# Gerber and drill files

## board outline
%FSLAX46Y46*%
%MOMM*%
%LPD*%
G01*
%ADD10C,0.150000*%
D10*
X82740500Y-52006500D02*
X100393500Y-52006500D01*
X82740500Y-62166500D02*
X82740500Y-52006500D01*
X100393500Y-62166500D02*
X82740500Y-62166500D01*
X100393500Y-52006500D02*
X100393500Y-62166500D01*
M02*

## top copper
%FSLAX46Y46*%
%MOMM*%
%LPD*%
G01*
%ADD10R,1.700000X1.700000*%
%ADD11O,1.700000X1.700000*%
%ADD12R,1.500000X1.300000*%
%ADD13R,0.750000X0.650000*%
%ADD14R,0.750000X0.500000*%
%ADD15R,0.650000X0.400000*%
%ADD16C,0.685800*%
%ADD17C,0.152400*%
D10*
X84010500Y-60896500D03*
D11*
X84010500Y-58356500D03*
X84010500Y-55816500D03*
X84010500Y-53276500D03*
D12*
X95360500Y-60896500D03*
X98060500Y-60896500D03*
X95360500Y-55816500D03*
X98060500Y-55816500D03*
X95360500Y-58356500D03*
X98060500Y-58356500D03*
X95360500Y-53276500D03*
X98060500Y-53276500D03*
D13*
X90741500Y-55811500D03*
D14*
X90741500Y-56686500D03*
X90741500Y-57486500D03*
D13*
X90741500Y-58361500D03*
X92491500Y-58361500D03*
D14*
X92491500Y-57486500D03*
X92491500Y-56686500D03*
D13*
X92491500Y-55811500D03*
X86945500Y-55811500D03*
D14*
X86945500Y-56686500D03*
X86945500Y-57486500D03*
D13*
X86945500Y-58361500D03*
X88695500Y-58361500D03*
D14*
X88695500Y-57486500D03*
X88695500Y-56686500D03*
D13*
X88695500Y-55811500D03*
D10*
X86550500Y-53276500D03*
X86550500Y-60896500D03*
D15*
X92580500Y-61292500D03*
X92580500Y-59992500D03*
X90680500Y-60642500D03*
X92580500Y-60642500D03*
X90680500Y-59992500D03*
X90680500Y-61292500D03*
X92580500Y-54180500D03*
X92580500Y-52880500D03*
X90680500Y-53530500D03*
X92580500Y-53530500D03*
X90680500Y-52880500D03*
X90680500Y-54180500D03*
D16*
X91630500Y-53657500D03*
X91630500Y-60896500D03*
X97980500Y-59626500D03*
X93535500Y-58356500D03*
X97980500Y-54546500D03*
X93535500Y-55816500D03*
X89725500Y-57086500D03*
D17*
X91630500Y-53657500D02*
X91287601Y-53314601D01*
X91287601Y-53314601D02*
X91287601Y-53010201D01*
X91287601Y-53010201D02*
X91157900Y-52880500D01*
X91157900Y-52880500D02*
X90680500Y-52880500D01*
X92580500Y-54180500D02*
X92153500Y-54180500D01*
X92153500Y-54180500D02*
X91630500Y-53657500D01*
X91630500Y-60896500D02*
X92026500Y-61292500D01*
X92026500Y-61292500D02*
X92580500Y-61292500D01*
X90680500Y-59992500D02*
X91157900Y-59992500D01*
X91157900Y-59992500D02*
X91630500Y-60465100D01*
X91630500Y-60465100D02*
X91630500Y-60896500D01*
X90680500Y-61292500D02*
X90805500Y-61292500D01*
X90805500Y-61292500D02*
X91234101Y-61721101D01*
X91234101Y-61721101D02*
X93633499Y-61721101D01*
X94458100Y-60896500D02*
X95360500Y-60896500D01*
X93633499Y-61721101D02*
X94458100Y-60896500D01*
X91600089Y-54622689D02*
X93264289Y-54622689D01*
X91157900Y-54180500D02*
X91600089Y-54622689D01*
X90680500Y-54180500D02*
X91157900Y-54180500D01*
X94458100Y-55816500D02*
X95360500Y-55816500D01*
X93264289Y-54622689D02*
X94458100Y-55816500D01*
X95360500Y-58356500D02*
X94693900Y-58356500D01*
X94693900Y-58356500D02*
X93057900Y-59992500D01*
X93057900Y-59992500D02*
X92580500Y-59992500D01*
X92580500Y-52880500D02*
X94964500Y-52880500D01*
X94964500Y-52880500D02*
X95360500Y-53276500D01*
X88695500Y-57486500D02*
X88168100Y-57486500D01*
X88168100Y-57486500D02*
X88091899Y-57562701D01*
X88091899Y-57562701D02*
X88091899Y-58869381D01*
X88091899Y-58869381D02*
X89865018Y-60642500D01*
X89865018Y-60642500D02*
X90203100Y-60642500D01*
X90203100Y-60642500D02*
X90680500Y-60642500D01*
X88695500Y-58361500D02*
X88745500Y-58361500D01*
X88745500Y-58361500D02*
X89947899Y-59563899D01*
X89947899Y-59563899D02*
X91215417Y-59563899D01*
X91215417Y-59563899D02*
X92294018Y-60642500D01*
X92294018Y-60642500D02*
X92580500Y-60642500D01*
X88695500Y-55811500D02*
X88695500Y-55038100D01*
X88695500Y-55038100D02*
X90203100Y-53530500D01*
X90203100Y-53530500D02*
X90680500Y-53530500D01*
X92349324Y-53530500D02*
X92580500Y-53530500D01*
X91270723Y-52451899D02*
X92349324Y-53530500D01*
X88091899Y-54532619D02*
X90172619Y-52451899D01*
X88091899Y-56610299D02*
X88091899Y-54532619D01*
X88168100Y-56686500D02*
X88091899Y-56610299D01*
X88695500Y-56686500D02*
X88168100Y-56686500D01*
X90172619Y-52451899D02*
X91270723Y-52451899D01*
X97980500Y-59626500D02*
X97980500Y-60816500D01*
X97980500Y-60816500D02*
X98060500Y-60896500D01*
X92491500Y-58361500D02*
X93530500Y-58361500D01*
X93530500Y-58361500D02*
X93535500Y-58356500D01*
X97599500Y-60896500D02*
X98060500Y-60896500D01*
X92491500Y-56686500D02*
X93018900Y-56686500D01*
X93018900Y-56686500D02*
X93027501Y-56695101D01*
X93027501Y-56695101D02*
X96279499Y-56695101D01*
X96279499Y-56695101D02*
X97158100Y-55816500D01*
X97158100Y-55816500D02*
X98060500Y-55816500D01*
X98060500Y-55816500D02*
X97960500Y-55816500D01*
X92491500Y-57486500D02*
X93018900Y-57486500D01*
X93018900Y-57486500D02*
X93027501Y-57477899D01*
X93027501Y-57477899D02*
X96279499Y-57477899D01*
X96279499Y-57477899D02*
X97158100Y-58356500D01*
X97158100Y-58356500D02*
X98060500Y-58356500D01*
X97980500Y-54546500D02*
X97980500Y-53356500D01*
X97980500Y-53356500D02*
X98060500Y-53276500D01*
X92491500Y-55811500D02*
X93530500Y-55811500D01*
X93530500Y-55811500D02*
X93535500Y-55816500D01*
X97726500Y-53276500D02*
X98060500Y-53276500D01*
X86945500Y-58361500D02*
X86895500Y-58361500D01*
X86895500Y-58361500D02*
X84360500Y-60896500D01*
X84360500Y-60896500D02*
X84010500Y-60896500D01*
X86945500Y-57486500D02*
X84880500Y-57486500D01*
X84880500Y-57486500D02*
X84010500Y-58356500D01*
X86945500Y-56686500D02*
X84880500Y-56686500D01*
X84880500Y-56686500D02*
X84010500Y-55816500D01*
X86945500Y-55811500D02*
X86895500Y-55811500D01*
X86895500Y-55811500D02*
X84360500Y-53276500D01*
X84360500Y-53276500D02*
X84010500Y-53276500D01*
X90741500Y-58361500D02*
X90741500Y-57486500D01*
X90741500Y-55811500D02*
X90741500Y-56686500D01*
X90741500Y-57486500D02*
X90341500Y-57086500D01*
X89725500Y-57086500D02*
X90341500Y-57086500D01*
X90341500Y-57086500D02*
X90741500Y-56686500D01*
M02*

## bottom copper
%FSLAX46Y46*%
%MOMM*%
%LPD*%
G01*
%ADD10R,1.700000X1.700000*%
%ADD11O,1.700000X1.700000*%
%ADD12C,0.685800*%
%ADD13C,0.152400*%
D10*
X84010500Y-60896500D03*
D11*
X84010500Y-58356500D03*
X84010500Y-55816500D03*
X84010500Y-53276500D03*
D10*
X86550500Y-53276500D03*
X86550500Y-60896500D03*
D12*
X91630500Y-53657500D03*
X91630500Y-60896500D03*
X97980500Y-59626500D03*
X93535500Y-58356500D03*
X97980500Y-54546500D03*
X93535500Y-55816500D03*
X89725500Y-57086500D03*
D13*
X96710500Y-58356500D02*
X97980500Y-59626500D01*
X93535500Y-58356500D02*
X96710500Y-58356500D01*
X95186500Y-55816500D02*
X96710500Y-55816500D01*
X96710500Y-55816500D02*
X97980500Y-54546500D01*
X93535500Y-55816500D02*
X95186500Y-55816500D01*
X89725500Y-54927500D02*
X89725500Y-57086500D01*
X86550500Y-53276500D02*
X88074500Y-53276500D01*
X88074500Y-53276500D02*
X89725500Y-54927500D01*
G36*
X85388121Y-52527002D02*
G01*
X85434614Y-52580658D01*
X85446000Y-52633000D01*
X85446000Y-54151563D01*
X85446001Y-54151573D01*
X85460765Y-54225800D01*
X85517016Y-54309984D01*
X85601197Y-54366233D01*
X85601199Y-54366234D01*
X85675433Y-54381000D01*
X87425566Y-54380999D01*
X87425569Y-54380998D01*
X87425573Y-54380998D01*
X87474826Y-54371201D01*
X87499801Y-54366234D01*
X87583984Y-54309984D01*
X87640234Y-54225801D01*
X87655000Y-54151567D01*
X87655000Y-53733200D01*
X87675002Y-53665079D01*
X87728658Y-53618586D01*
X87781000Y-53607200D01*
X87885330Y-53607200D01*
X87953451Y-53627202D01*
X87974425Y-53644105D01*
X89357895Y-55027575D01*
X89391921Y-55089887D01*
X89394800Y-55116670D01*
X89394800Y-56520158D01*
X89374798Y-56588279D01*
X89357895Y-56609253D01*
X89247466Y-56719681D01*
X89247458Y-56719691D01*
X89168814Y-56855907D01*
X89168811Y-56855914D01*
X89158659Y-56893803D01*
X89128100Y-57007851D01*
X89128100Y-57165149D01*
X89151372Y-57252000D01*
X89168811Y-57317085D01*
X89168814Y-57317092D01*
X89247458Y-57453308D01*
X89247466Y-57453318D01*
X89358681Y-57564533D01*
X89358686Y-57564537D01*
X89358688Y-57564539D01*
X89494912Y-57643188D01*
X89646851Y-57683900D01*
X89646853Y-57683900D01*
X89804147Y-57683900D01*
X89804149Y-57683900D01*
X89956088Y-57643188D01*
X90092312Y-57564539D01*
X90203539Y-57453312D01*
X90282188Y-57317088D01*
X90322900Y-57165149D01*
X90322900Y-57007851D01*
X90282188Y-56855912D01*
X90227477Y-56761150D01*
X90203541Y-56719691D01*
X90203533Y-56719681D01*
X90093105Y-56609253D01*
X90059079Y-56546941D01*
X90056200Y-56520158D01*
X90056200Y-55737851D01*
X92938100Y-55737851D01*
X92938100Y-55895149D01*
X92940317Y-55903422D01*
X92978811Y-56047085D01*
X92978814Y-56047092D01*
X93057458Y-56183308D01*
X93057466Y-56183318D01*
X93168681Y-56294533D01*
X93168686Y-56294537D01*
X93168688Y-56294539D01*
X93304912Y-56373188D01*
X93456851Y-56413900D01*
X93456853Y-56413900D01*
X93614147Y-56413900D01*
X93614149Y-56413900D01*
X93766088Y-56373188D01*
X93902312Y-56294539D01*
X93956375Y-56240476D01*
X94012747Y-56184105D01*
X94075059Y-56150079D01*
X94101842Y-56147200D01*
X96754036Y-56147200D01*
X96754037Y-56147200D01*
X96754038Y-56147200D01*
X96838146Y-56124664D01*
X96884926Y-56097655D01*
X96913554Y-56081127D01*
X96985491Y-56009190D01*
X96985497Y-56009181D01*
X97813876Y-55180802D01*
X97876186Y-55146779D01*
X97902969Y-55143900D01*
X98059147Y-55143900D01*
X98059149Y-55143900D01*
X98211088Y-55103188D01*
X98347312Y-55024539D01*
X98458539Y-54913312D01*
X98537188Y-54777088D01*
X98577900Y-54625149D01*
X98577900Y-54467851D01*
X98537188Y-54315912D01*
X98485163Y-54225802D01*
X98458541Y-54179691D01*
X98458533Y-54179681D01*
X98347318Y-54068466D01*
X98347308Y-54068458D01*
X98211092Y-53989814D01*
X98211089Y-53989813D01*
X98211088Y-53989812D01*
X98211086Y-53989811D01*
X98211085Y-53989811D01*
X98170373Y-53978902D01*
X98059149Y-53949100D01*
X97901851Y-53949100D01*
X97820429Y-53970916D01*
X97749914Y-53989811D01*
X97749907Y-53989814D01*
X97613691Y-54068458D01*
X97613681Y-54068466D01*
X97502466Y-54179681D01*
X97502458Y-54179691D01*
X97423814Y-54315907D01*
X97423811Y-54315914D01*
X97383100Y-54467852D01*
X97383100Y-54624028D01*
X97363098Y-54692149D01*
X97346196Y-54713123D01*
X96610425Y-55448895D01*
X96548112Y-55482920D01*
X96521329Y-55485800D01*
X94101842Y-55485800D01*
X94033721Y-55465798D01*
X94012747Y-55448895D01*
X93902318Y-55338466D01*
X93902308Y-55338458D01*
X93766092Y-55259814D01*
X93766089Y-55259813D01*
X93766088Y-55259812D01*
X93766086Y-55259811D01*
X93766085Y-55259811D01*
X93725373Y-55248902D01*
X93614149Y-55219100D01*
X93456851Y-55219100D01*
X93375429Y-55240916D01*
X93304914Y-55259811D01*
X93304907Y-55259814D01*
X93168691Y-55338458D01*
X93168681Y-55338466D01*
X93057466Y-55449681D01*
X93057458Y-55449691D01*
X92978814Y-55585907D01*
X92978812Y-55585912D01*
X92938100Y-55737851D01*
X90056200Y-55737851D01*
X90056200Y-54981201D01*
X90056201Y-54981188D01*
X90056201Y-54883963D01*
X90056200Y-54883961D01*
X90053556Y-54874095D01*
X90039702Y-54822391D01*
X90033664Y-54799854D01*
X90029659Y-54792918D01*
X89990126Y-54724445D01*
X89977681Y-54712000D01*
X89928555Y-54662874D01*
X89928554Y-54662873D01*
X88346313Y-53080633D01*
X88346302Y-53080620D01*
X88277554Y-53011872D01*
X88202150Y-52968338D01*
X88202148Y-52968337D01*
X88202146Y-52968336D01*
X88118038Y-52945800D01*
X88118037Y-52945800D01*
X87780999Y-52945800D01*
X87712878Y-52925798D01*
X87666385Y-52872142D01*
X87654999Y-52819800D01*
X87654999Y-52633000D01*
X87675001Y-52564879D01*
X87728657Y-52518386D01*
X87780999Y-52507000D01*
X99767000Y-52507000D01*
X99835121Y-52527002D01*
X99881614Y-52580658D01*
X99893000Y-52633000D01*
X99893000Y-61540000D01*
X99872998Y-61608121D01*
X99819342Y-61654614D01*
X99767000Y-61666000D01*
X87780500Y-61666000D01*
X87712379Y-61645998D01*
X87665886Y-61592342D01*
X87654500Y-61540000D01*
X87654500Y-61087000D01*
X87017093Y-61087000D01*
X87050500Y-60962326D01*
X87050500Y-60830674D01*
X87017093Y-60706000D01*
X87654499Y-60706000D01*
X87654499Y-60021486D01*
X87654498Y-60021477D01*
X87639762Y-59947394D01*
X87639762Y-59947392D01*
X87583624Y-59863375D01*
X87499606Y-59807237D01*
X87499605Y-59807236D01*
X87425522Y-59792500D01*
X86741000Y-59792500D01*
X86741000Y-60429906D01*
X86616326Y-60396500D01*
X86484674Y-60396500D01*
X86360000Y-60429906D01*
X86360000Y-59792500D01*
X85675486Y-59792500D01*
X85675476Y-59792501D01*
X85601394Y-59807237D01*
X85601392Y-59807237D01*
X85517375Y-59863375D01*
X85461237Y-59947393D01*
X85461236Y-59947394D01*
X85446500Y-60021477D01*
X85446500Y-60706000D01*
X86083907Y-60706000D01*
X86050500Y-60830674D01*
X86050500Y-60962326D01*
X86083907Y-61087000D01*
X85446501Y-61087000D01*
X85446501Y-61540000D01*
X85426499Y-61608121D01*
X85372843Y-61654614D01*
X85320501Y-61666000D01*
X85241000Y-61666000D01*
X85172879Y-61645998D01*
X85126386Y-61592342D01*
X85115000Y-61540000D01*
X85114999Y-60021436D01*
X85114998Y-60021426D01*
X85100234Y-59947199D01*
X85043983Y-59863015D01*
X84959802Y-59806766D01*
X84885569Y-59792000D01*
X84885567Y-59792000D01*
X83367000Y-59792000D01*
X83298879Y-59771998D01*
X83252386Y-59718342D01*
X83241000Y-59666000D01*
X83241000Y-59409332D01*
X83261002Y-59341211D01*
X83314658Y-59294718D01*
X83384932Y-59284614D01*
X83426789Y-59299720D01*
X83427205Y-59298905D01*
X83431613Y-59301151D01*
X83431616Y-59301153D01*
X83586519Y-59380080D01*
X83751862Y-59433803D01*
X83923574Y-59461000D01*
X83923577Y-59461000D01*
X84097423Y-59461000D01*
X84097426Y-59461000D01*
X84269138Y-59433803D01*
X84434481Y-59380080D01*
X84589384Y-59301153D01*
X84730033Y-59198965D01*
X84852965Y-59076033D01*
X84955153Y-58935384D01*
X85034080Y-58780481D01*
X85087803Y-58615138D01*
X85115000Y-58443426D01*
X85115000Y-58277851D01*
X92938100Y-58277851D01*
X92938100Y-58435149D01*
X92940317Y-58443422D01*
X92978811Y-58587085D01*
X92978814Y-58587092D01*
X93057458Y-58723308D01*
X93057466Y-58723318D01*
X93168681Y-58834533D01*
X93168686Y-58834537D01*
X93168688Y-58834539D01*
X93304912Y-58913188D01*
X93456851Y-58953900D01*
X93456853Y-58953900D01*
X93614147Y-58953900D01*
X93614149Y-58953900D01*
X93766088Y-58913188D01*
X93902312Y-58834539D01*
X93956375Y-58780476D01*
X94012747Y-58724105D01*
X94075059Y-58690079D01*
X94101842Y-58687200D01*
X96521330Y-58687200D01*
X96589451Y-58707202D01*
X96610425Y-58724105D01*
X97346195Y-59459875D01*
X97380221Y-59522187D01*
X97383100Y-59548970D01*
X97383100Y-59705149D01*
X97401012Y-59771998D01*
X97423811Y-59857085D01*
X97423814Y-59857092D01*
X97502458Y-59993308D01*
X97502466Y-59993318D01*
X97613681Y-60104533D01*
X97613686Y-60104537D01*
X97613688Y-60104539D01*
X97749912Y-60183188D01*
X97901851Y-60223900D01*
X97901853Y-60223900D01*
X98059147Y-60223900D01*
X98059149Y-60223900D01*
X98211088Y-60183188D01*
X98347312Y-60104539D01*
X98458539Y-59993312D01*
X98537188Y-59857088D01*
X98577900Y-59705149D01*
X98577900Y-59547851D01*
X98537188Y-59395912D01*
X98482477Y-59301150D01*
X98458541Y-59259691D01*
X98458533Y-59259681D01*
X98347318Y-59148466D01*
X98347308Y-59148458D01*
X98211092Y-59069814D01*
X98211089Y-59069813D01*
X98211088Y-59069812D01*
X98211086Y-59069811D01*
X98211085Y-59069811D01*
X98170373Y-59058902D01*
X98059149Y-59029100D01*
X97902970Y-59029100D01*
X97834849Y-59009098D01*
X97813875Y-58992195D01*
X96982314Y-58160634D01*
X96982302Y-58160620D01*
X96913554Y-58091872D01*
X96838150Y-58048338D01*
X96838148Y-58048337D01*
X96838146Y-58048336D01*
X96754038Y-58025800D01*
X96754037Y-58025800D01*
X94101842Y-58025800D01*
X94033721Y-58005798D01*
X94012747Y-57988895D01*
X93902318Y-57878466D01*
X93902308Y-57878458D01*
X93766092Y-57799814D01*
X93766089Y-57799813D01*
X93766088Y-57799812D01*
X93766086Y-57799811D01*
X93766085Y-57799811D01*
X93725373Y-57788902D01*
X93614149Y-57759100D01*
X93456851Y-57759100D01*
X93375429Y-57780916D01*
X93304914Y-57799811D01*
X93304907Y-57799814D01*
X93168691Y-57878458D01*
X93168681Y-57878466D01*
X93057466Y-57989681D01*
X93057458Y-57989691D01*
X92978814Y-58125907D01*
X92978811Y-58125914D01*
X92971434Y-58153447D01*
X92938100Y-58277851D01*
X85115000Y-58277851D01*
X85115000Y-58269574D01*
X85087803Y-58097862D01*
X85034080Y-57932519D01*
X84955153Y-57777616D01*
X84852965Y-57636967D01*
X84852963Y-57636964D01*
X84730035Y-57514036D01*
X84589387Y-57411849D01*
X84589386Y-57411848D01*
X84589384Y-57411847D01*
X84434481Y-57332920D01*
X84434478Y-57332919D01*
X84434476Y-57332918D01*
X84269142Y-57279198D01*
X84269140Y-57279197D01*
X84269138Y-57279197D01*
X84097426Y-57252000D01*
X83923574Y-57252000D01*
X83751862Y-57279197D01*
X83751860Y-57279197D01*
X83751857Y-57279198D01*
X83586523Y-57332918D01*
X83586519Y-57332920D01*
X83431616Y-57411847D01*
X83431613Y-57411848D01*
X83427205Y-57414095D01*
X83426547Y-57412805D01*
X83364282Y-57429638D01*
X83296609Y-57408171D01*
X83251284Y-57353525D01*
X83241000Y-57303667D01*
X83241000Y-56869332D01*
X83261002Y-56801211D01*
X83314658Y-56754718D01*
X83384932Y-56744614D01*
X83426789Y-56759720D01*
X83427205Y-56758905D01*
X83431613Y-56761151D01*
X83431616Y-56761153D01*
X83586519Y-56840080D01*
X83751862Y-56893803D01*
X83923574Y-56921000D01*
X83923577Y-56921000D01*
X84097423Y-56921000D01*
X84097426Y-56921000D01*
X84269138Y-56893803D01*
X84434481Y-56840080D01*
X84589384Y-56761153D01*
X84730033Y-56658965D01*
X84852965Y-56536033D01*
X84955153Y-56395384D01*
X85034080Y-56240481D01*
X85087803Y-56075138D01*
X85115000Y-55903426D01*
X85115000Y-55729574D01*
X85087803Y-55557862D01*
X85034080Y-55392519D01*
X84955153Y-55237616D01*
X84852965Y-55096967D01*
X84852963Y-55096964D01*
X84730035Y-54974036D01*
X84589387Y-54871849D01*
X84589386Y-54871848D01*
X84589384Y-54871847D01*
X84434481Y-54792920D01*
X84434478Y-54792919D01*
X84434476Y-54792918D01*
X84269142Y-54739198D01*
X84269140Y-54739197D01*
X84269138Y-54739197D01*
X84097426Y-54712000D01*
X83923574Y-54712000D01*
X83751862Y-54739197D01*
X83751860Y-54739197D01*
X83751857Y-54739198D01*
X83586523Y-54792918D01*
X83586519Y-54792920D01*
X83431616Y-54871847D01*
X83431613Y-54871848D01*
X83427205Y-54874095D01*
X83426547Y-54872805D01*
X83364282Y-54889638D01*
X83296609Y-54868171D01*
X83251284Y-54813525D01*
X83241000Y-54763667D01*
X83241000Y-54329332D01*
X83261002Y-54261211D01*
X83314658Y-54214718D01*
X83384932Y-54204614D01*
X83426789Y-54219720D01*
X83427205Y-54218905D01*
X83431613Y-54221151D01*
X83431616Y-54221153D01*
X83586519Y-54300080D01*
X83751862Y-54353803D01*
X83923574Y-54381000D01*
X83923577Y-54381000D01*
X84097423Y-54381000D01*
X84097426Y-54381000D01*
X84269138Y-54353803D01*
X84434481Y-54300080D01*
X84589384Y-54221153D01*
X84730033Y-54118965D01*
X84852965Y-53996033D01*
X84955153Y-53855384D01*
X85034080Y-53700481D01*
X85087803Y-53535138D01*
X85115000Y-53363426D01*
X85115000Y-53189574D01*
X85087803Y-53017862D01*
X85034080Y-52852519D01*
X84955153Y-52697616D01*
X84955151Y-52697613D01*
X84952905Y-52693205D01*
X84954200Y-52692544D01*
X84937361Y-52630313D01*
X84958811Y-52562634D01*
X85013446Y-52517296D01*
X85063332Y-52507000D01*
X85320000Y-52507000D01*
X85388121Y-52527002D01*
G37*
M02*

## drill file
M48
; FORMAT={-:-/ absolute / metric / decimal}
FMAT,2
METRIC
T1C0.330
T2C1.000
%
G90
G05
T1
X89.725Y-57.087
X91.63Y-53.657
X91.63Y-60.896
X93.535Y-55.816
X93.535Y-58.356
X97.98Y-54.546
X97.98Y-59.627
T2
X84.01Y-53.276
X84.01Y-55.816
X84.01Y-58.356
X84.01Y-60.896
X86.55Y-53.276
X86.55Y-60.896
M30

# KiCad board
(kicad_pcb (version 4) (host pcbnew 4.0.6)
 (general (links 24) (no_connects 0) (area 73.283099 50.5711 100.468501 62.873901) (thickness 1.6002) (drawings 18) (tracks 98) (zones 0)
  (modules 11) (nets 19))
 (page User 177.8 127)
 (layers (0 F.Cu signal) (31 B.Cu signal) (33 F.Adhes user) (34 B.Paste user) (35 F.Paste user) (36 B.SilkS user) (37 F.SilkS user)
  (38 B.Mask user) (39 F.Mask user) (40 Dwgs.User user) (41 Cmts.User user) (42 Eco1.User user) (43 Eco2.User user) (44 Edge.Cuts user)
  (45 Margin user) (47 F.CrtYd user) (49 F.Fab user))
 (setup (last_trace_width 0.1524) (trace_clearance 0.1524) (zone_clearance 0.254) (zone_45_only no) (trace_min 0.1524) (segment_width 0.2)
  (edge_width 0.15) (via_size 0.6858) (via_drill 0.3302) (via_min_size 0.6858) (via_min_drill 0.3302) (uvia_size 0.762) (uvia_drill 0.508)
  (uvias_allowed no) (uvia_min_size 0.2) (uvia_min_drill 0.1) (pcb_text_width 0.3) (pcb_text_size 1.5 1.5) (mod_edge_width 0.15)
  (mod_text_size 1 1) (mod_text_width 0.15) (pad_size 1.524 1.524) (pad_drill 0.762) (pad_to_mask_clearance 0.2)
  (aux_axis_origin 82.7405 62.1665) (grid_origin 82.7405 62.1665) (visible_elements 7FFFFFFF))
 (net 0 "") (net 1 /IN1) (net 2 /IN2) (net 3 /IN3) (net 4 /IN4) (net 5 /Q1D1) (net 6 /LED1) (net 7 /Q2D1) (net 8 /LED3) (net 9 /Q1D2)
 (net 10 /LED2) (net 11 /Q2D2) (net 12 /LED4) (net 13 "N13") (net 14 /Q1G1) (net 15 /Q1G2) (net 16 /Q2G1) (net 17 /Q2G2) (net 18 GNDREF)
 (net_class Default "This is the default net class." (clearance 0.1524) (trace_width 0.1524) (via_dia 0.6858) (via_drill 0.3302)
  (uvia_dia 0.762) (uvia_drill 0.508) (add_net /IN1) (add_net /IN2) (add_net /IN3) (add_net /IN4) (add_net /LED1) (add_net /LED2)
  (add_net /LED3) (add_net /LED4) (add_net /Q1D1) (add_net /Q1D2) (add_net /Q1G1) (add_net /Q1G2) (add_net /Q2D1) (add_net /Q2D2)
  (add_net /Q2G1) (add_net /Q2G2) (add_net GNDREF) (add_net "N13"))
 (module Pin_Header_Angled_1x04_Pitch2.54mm (layer F.Cu) (at 84.0105 60.8965 180)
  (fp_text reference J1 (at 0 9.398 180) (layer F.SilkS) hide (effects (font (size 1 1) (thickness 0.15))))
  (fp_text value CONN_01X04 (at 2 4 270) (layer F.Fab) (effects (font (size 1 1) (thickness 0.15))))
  (pad 1 thru_hole rect (at 0 0 180) (size 1.7 1.7) (drill 1) (layers *.Cu *.Mask) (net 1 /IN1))
  (pad 2 thru_hole oval (at 0 2.54 180) (size 1.7 1.7) (drill 1) (layers *.Cu *.Mask) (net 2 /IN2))
  (pad 3 thru_hole oval (at 0 5.08 180) (size 1.7 1.7) (drill 1) (layers *.Cu *.Mask) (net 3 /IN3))
  (pad 4 thru_hole oval (at 0 7.62 180) (size 1.7 1.7) (drill 1) (layers *.Cu *.Mask) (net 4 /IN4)))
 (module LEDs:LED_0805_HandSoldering (layer F.Cu) (at 96.7105 60.8965)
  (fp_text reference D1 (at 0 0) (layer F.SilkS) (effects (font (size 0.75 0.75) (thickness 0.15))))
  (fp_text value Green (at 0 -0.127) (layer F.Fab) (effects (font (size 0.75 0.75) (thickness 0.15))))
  (pad 1 smd rect (at -1.35 0) (size 1.5 1.3) (layers F.Cu F.Paste F.Mask) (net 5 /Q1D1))
  (pad 2 smd rect (at 1.35 0) (size 1.5 1.3) (layers F.Cu F.Paste F.Mask) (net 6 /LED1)))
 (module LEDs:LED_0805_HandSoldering (layer F.Cu) (at 96.7105 55.8165)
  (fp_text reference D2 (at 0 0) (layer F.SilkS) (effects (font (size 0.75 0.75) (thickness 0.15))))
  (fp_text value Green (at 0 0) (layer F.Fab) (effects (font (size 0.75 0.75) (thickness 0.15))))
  (pad 1 smd rect (at -1.35 0) (size 1.5 1.3) (layers F.Cu F.Paste F.Mask) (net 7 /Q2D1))
  (pad 2 smd rect (at 1.35 0) (size 1.5 1.3) (layers F.Cu F.Paste F.Mask) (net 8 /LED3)))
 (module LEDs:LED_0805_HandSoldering (layer F.Cu) (at 96.7105 58.3565)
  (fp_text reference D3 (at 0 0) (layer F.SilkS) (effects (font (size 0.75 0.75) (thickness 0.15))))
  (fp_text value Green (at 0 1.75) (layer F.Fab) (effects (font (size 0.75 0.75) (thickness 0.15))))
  (pad 1 smd rect (at -1.35 0) (size 1.5 1.3) (layers F.Cu F.Paste F.Mask) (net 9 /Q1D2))
  (pad 2 smd rect (at 1.35 0) (size 1.5 1.3) (layers F.Cu F.Paste F.Mask) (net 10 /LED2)))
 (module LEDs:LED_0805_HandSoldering (layer F.Cu) (at 96.7105 53.2765)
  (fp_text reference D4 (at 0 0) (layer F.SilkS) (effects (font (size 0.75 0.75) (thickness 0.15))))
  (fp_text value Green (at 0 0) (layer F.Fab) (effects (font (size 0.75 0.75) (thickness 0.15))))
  (pad 1 smd rect (at -1.35 0) (size 1.5 1.3) (layers F.Cu F.Paste F.Mask) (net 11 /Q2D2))
  (pad 2 smd rect (at 1.35 0) (size 1.5 1.3) (layers F.Cu F.Paste F.Mask) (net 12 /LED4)))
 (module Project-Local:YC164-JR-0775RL (layer F.Cu) (at 91.6165 57.0865)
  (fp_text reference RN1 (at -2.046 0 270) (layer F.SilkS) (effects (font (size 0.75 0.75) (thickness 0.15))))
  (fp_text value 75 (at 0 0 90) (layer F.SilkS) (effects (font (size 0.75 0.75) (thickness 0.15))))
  (pad 1 smd rect (at -0.875 -1.275) (size 0.75 0.65) (layers F.Cu F.Paste F.Mask) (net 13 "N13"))
  (pad 2 smd rect (at -0.875 -0.4) (size 0.75 0.5) (layers F.Cu F.Paste F.Mask) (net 13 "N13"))
  (pad 3 smd rect (at -0.875 0.4) (size 0.75 0.5) (layers F.Cu F.Paste F.Mask) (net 13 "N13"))
  (pad 4 smd rect (at -0.875 1.275) (size 0.75 0.65) (layers F.Cu F.Paste F.Mask) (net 13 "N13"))
  (pad 5 smd rect (at 0.875 1.275) (size 0.75 0.65) (layers F.Cu F.Paste F.Mask) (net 6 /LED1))
  (pad 6 smd rect (at 0.875 0.4) (size 0.75 0.5) (layers F.Cu F.Paste F.Mask) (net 10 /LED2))
  (pad 7 smd rect (at 0.875 -0.4) (size 0.75 0.5) (layers F.Cu F.Paste F.Mask) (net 8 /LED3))
  (pad 8 smd rect (at 0.875 -1.275) (size 0.75 0.65) (layers F.Cu F.Paste F.Mask) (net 12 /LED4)))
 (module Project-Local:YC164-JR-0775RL (layer F.Cu) (at 87.8205 57.0865)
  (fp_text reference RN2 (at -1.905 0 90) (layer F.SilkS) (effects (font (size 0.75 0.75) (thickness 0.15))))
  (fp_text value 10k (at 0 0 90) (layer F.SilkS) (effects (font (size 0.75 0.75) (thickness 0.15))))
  (pad 1 smd rect (at -0.875 -1.275) (size 0.75 0.65) (layers F.Cu F.Paste F.Mask) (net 4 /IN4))
  (pad 2 smd rect (at -0.875 -0.4) (size 0.75 0.5) (layers F.Cu F.Paste F.Mask) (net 3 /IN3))
  (pad 3 smd rect (at -0.875 0.4) (size 0.75 0.5) (layers F.Cu F.Paste F.Mask) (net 2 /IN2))
  (pad 4 smd rect (at -0.875 1.275) (size 0.75 0.65) (layers F.Cu F.Paste F.Mask) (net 1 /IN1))
  (pad 5 smd rect (at 0.875 1.275) (size 0.75 0.65) (layers F.Cu F.Paste F.Mask) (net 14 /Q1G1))
  (pad 6 smd rect (at 0.875 0.4) (size 0.75 0.5) (layers F.Cu F.Paste F.Mask) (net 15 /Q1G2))
  (pad 7 smd rect (at 0.875 -0.4) (size 0.75 0.5) (layers F.Cu F.Paste F.Mask) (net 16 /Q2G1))
  (pad 8 smd rect (at 0.875 -1.275) (size 0.75 0.65) (layers F.Cu F.Paste F.Mask) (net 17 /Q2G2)))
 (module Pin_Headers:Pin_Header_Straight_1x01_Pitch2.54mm (layer F.Cu) (at 86.5505 53.2765)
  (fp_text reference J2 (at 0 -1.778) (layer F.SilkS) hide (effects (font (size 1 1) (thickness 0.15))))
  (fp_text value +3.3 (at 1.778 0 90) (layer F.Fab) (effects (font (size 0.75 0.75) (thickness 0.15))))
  (pad 1 thru_hole rect (at 0 0) (size 1.7 1.7) (drill 1) (layers *.Cu *.Mask) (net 13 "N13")))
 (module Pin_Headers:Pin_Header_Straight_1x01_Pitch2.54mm (layer F.Cu) (at 86.5505 60.8965)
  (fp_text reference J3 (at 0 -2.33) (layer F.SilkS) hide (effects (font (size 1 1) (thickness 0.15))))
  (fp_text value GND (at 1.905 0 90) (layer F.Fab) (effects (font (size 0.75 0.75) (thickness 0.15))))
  (pad 1 thru_hole rect (at 0 0) (size 1.7 1.7) (drill 1) (layers *.Cu *.Mask) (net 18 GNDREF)))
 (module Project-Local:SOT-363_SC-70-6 (layer F.Cu) (at 91.6305 60.6425 180)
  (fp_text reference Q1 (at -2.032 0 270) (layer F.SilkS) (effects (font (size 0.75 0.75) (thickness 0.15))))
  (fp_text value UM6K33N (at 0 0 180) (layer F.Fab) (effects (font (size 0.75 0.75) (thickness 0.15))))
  (pad 1 smd rect (at -0.95 -0.65 180) (size 0.65 0.4) (layers F.Cu F.Paste F.Mask) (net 18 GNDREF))
  (pad 3 smd rect (at -0.95 0.65 180) (size 0.65 0.4) (layers F.Cu F.Paste F.Mask) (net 9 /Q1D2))
  (pad 5 smd rect (at 0.95 0 180) (size 0.65 0.4) (layers F.Cu F.Paste F.Mask) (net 15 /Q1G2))
  (pad 2 smd rect (at -0.95 0 180) (size 0.65 0.4) (layers F.Cu F.Paste F.Mask) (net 14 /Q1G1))
  (pad 4 smd rect (at 0.95 0.65 180) (size 0.65 0.4) (layers F.Cu F.Paste F.Mask) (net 18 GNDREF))
  (pad 6 smd rect (at 0.95 -0.65 180) (size 0.65 0.4) (layers F.Cu F.Paste F.Mask) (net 5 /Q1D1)))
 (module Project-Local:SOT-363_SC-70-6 (layer F.Cu) (at 91.6305 53.5305 180)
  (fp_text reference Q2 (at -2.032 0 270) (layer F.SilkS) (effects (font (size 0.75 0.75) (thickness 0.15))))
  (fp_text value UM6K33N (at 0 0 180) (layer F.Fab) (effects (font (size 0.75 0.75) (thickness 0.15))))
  (pad 1 smd rect (at -0.95 -0.65 180) (size 0.65 0.4) (layers F.Cu F.Paste F.Mask) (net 18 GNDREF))
  (pad 3 smd rect (at -0.95 0.65 180) (size 0.65 0.4) (layers F.Cu F.Paste F.Mask) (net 11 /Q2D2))
  (pad 5 smd rect (at 0.95 0 180) (size 0.65 0.4) (layers F.Cu F.Paste F.Mask) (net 17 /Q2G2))
  (pad 2 smd rect (at -0.95 0 180) (size 0.65 0.4) (layers F.Cu F.Paste F.Mask) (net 16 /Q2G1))
  (pad 4 smd rect (at 0.95 0.65 180) (size 0.65 0.4) (layers F.Cu F.Paste F.Mask) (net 18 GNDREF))
  (pad 6 smd rect (at 0.95 -0.65 180) (size 0.65 0.4) (layers F.Cu F.Paste F.Mask) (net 7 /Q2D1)))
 (gr_line (start 82.7405 52.0065) (end 100.3935 52.0065) (layer Edge.Cuts) (width 0.15))
 (gr_line (start 82.7405 62.1665) (end 82.7405 52.0065) (layer Edge.Cuts) (width 0.15))
 (gr_line (start 100.3935 62.1665) (end 82.7405 62.1665) (layer Edge.Cuts) (width 0.15))
 (gr_line (start 100.3935 52.0065) (end 100.3935 62.1665) (layer Edge.Cuts) (width 0.15))
 (segment (start 91.6305 53.6575) (end 91.287601 53.314601) (width 0.1524) (layer F.Cu) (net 18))
 (segment (start 91.287601 53.314601) (end 91.287601 53.010201) (width 0.1524) (layer F.Cu) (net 18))
 (segment (start 91.287601 53.010201) (end 91.1579 52.8805) (width 0.1524) (layer F.Cu) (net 18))
 (segment (start 91.1579 52.8805) (end 90.6805 52.8805) (width 0.1524) (layer F.Cu) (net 18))
 (segment (start 92.5805 54.1805) (end 92.1535 54.1805) (width 0.1524) (layer F.Cu) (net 18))
 (segment (start 92.1535 54.1805) (end 91.6305 53.6575) (width 0.1524) (layer F.Cu) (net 18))
 (via (at 91.6305 53.6575) (size 0.6858) (drill 0.3302) (layers F.Cu B.Cu) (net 18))
 (segment (start 91.6305 60.8965) (end 92.0265 61.2925) (width 0.1524) (layer F.Cu) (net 18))
 (segment (start 92.0265 61.2925) (end 92.5805 61.2925) (width 0.1524) (layer F.Cu) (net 18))
 (via (at 91.6305 60.8965) (size 0.6858) (drill 0.3302) (layers F.Cu B.Cu) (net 18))
 (segment (start 90.6805 59.9925) (end 91.1579 59.9925) (width 0.1524) (layer F.Cu) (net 18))
 (segment (start 91.1579 59.9925) (end 91.6305 60.4651) (width 0.1524) (layer F.Cu) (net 18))
 (segment (start 91.6305 60.4651) (end 91.6305 60.8965) (width 0.1524) (layer F.Cu) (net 18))
 (segment (start 90.6805 61.2925) (end 90.8055 61.2925) (width 0.1524) (layer F.Cu) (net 5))
 (segment (start 90.8055 61.2925) (end 91.234101 61.721101) (width 0.1524) (layer F.Cu) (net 5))
 (segment (start 91.234101 61.721101) (end 93.633499 61.721101) (width 0.1524) (layer F.Cu) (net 5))
 (segment (start 94.4581 60.8965) (end 95.3605 60.8965) (width 0.1524) (layer F.Cu) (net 5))
 (segment (start 93.633499 61.721101) (end 94.4581 60.8965) (width 0.1524) (layer F.Cu) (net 5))
 (segment (start 91.600089 54.622689) (end 93.264289 54.622689) (width 0.1524) (layer F.Cu) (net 7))
 (segment (start 91.1579 54.1805) (end 91.600089 54.622689) (width 0.1524) (layer F.Cu) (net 7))
 (segment (start 90.6805 54.1805) (end 91.1579 54.1805) (width 0.1524) (layer F.Cu) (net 7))
 (segment (start 94.4581 55.8165) (end 95.3605 55.8165) (width 0.1524) (layer F.Cu) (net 7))
 (segment (start 93.264289 54.622689) (end 94.4581 55.8165) (width 0.1524) (layer F.Cu) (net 7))
 (segment (start 95.3605 58.3565) (end 94.6939 58.3565) (width 0.1524) (layer F.Cu) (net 9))
 (segment (start 94.6939 58.3565) (end 93.0579 59.9925) (width 0.1524) (layer F.Cu) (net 9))
 (segment (start 93.0579 59.9925) (end 92.5805 59.9925) (width 0.1524) (layer F.Cu) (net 9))
 (segment (start 92.5805 52.8805) (end 94.9645 52.8805) (width 0.1524) (layer F.Cu) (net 11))
 (segment (start 94.9645 52.8805) (end 95.3605 53.2765) (width 0.1524) (layer F.Cu) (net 11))
 (segment (start 88.6955 57.4865) (end 88.1681 57.4865) (width 0.1524) (layer F.Cu) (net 15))
 (segment (start 88.1681 57.4865) (end 88.091899 57.562701) (width 0.1524) (layer F.Cu) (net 15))
 (segment (start 88.091899 57.562701) (end 88.091899 58.869381) (width 0.1524) (layer F.Cu) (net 15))
 (segment (start 88.091899 58.869381) (end 89.865018 60.6425) (width 0.1524) (layer F.Cu) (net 15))
 (segment (start 89.865018 60.6425) (end 90.2031 60.6425) (width 0.1524) (layer F.Cu) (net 15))
 (segment (start 90.2031 60.6425) (end 90.6805 60.6425) (width 0.1524) (layer F.Cu) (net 15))
 (segment (start 88.6955 58.3615) (end 88.7455 58.3615) (width 0.1524) (layer F.Cu) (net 14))
 (segment (start 88.7455 58.3615) (end 89.947899 59.563899) (width 0.1524) (layer F.Cu) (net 14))
 (segment (start 89.947899 59.563899) (end 91.215417 59.563899) (width 0.1524) (layer F.Cu) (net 14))
 (segment (start 91.215417 59.563899) (end 92.294018 60.6425) (width 0.1524) (layer F.Cu) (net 14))
 (segment (start 92.294018 60.6425) (end 92.5805 60.6425) (width 0.1524) (layer F.Cu) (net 14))
 (segment (start 88.6955 55.8115) (end 88.6955 55.0381) (width 0.1524) (layer F.Cu) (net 17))
 (segment (start 88.6955 55.0381) (end 90.2031 53.5305) (width 0.1524) (layer F.Cu) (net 17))
 (segment (start 90.2031 53.5305) (end 90.6805 53.5305) (width 0.1524) (layer F.Cu) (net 17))
 (segment (start 92.349324 53.5305) (end 92.5805 53.5305) (width 0.1524) (layer F.Cu) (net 16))
 (segment (start 91.270723 52.451899) (end 92.349324 53.5305) (width 0.1524) (layer F.Cu) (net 16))
 (segment (start 88.091899 54.532619) (end 90.172619 52.451899) (width 0.1524) (layer F.Cu) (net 16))
 (segment (start 88.091899 56.610299) (end 88.091899 54.532619) (width 0.1524) (layer F.Cu) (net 16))
 (segment (start 88.1681 56.6865) (end 88.091899 56.610299) (width 0.1524) (layer F.Cu) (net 16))
 (segment (start 88.6955 56.6865) (end 88.1681 56.6865) (width 0.1524) (layer F.Cu) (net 16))
 (segment (start 90.172619 52.451899) (end 91.270723 52.451899) (width 0.1524) (layer F.Cu) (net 16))
 (segment (start 97.9805 59.6265) (end 97.9805 60.8165) (width 0.1524) (layer F.Cu) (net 6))
 (segment (start 97.9805 60.8165) (end 98.0605 60.8965) (width 0.1524) (layer F.Cu) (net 6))
 (via (at 97.9805 59.6265) (size 0.6858) (drill 0.3302) (layers F.Cu B.Cu) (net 6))
 (segment (start 96.7105 58.3565) (end 97.9805 59.6265) (width 0.1524) (layer B.Cu) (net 6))
 (segment (start 93.5355 58.3565) (end 96.7105 58.3565) (width 0.1524) (layer B.Cu) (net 6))
 (segment (start 92.4915 58.3615) (end 93.5305 58.3615) (width 0.1524) (layer F.Cu) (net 6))
 (segment (start 93.5305 58.3615) (end 93.5355 58.3565) (width 0.1524) (layer F.Cu) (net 6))
 (via (at 93.5355 58.3565) (size 0.6858) (drill 0.3302) (layers F.Cu B.Cu) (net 6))
 (segment (start 97.5995 60.8965) (end 98.0605 60.8965) (width 0.1524) (layer F.Cu) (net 6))
 (segment (start 92.4915 56.6865) (end 93.0189 56.6865) (width 0.1524) (layer F.Cu) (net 8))
 (segment (start 93.0189 56.6865) (end 93.027501 56.695101) (width 0.1524) (layer F.Cu) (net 8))
 (segment (start 93.027501 56.695101) (end 96.279499 56.695101) (width 0.1524) (layer F.Cu) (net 8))
 (segment (start 96.279499 56.695101) (end 97.1581 55.8165) (width 0.1524) (layer F.Cu) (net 8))
 (segment (start 97.1581 55.8165) (end 98.0605 55.8165) (width 0.1524) (layer F.Cu) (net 8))
 (segment (start 98.0605 55.8165) (end 97.9605 55.8165) (width 0.1524) (layer F.Cu) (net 8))
 (segment (start 92.4915 57.4865) (end 93.0189 57.4865) (width 0.1524) (layer F.Cu) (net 10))
 (segment (start 93.0189 57.4865) (end 93.027501 57.477899) (width 0.1524) (layer F.Cu) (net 10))
 (segment (start 93.027501 57.477899) (end 96.279499 57.477899) (width 0.1524) (layer F.Cu) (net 10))
 (segment (start 96.279499 57.477899) (end 97.1581 58.3565) (width 0.1524) (layer F.Cu) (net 10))
 (segment (start 97.1581 58.3565) (end 98.0605 58.3565) (width 0.1524) (layer F.Cu) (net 10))
 (segment (start 97.9805 54.5465) (end 97.9805 53.3565) (width 0.1524) (layer F.Cu) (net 12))
 (segment (start 97.9805 53.3565) (end 98.0605 53.2765) (width 0.1524) (layer F.Cu) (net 12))
 (segment (start 95.1865 55.8165) (end 96.7105 55.8165) (width 0.1524) (layer B.Cu) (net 12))
 (segment (start 96.7105 55.8165) (end 97.9805 54.5465) (width 0.1524) (layer B.Cu) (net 12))
 (via (at 97.9805 54.5465) (size 0.6858) (drill 0.3302) (layers F.Cu B.Cu) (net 12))
 (segment (start 93.5355 55.8165) (end 95.1865 55.8165) (width 0.1524) (layer B.Cu) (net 12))
 (segment (start 92.4915 55.8115) (end 93.5305 55.8115) (width 0.1524) (layer F.Cu) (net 12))
 (segment (start 93.5305 55.8115) (end 93.5355 55.8165) (width 0.1524) (layer F.Cu) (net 12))
 (via (at 93.5355 55.8165) (size 0.6858) (drill 0.3302) (layers F.Cu B.Cu) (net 12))
 (segment (start 97.7265 53.2765) (end 98.0605 53.2765) (width 0.1524) (layer F.Cu) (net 12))
 (segment (start 86.9455 58.3615) (end 86.8955 58.3615) (width 0.1524) (layer F.Cu) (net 1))
 (segment (start 86.8955 58.3615) (end 84.3605 60.8965) (width 0.1524) (layer F.Cu) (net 1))
 (segment (start 84.3605 60.8965) (end 84.0105 60.8965) (width 0.1524) (layer F.Cu) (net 1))
 (segment (start 86.9455 57.4865) (end 84.8805 57.4865) (width 0.1524) (layer F.Cu) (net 2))
 (segment (start 84.8805 57.4865) (end 84.0105 58.3565) (width 0.1524) (layer F.Cu) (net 2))
 (segment (start 86.9455 56.6865) (end 84.8805 56.6865) (width 0.1524) (layer F.Cu) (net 3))
 (segment (start 84.8805 56.6865) (end 84.0105 55.8165) (width 0.1524) (layer F.Cu) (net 3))
 (segment (start 86.9455 55.8115) (end 86.8955 55.8115) (width 0.1524) (layer F.Cu) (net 4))
 (segment (start 86.8955 55.8115) (end 84.3605 53.2765) (width 0.1524) (layer F.Cu) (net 4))
 (segment (start 84.3605 53.2765) (end 84.0105 53.2765) (width 0.1524) (layer F.Cu) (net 4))
 (segment (start 90.7415 58.3615) (end 90.7415 57.4865) (width 0.1524) (layer F.Cu) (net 13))
 (segment (start 90.7415 55.8115) (end 90.7415 56.6865) (width 0.1524) (layer F.Cu) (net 13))
 (segment (start 90.7415 57.4865) (end 90.3415 57.0865) (width 0.1524) (layer F.Cu) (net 13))
 (segment (start 89.7255 57.0865) (end 90.3415 57.0865) (width 0.1524) (layer F.Cu) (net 13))
 (segment (start 90.3415 57.0865) (end 90.7415 56.6865) (width 0.1524) (layer F.Cu) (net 13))
 (segment (start 89.7255 54.9275) (end 89.7255 57.0865) (width 0.1524) (layer B.Cu) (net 13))
 (via (at 89.7255 57.0865) (size 0.6858) (drill 0.3302) (layers F.Cu B.Cu) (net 13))
 (segment (start 86.5505 53.2765) (end 88.0745 53.2765) (width 0.1524) (layer B.Cu) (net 13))
 (segment (start 88.0745 53.2765) (end 89.7255 54.9275) (width 0.1524) (layer B.Cu) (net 13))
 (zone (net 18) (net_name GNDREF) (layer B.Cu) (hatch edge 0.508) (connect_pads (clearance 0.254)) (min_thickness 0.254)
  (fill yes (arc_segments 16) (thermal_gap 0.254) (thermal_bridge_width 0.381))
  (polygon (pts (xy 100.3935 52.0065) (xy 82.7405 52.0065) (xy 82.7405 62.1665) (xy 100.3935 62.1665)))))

